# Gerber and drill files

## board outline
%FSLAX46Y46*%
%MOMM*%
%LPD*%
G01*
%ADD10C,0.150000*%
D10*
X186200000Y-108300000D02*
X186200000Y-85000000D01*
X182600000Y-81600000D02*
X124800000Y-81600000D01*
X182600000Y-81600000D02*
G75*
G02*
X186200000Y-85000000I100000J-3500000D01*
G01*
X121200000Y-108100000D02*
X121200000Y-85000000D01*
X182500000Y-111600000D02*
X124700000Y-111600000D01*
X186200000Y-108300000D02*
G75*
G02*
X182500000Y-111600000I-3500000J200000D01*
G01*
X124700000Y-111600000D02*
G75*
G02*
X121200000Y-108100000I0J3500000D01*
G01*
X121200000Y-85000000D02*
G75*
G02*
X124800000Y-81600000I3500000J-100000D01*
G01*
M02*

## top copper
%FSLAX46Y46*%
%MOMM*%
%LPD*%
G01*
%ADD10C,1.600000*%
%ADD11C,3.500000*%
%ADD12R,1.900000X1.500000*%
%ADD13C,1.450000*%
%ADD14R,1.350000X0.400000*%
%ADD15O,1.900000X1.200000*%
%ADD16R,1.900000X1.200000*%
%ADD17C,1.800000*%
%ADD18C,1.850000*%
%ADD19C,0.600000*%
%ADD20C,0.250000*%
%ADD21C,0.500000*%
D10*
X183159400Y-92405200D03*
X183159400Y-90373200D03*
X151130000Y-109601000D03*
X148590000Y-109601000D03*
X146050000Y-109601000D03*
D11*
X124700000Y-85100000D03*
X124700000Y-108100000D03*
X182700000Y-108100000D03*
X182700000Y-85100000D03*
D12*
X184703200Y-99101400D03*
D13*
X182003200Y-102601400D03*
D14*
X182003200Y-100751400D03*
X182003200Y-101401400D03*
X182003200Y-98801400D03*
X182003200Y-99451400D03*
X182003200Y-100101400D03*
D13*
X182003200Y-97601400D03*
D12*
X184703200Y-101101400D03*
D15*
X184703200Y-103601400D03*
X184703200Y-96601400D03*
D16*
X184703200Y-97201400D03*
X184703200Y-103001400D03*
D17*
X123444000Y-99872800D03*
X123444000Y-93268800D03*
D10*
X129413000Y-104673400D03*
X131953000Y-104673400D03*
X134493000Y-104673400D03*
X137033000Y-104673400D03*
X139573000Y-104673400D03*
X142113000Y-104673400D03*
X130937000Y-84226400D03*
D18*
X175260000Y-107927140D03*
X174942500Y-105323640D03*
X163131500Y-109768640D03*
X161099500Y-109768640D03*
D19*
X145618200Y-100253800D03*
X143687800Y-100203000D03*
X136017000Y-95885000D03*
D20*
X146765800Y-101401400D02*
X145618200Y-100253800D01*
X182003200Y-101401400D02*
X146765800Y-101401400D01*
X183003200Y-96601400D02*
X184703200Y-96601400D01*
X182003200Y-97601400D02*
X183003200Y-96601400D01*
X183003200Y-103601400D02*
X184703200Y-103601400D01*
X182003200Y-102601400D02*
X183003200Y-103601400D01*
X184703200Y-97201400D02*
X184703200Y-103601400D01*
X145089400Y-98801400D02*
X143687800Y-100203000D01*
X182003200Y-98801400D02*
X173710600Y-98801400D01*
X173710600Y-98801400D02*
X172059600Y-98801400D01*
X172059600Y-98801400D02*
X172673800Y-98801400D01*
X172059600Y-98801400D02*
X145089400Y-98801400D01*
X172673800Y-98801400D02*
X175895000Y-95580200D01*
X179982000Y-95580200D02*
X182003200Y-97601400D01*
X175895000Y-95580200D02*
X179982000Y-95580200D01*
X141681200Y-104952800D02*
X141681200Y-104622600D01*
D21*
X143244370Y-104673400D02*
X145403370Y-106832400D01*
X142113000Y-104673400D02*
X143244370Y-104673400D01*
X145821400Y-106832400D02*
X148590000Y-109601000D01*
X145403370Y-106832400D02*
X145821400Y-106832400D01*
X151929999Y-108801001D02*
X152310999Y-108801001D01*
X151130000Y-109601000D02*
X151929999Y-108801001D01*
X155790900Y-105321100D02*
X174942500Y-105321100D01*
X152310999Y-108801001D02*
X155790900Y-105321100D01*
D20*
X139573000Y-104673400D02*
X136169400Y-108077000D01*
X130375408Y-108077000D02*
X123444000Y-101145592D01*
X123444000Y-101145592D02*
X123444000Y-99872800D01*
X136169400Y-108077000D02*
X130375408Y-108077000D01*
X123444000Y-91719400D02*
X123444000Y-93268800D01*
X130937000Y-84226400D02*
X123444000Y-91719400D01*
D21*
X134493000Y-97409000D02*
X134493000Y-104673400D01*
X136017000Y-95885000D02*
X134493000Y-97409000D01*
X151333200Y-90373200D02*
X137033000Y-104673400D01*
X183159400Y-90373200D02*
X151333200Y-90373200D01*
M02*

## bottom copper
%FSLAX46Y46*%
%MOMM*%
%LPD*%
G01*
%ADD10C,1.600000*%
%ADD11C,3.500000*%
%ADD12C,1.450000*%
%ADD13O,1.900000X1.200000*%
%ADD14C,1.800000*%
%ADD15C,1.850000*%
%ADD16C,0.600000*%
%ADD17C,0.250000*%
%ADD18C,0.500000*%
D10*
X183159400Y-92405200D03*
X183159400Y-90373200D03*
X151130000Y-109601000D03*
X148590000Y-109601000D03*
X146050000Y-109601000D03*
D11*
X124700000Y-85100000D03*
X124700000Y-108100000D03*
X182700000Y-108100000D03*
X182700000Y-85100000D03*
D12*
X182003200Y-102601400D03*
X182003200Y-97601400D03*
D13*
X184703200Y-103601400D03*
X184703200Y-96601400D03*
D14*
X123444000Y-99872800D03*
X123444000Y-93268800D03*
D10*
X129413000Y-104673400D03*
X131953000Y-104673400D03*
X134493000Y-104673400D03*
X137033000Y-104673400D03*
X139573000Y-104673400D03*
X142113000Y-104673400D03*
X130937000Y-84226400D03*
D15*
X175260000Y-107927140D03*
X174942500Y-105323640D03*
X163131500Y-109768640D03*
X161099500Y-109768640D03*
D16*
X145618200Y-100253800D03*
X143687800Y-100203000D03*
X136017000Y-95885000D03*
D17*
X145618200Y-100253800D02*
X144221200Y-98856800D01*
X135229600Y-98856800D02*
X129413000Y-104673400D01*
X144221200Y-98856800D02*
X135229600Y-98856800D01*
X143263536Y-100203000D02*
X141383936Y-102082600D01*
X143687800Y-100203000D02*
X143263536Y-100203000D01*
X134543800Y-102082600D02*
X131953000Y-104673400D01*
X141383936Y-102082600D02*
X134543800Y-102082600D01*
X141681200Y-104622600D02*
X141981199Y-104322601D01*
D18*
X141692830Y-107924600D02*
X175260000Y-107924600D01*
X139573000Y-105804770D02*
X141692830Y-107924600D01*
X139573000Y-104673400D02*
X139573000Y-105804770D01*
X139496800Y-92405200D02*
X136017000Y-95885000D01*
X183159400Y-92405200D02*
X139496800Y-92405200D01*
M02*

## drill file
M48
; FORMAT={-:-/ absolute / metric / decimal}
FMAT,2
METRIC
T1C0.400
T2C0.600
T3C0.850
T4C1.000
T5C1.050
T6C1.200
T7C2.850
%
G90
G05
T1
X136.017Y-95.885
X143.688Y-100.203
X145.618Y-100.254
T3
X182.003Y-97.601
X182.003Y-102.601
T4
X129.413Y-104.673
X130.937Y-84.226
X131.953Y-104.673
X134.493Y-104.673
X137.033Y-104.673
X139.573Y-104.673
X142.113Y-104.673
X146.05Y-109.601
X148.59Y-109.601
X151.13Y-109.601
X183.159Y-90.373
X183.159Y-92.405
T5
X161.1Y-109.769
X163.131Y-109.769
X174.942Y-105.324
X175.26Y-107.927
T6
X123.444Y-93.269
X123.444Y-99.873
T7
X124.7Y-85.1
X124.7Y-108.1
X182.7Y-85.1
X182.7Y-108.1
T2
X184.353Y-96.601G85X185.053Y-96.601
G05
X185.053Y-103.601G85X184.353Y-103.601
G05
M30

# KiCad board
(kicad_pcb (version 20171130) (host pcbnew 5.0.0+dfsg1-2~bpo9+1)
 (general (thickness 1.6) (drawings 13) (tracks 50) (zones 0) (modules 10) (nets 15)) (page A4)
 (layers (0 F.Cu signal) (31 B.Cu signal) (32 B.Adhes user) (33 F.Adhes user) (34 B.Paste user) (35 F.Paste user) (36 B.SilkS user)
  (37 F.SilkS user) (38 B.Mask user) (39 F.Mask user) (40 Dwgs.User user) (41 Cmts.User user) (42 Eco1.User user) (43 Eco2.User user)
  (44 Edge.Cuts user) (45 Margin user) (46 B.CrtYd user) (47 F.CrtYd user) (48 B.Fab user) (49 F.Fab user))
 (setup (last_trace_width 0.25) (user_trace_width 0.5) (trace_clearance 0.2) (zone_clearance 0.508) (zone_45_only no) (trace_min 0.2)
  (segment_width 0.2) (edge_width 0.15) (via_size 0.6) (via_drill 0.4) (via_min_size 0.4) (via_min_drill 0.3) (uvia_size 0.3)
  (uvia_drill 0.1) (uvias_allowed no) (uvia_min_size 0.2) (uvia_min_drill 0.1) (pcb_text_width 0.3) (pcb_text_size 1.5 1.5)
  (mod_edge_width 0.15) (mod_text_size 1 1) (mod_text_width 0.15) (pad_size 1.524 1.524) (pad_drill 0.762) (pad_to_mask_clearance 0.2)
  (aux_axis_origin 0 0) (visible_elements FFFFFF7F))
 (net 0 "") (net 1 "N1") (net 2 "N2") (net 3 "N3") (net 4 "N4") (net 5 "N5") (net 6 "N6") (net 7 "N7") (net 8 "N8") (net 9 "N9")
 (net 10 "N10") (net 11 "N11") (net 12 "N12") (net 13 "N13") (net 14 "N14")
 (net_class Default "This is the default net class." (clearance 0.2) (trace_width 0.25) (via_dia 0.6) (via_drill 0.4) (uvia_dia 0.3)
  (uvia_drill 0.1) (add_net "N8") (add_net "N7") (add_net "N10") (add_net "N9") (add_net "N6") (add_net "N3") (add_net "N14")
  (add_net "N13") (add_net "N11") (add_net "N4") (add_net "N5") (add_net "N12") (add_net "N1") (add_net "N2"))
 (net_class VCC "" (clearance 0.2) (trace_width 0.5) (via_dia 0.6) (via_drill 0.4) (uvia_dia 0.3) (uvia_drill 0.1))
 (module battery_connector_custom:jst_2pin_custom (layer F.Cu) (at 183.1594 91.3892 90)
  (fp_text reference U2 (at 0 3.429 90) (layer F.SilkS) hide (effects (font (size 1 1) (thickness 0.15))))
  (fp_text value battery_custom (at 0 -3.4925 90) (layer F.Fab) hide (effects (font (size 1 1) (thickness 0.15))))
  (pad 1 thru_hole circle (at -1.016 0 90) (size 1.6 1.6) (drill 1) (layers *.Cu *.Mask) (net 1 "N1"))
  (pad 2 thru_hole circle (at 1.016 0 90) (size 1.6 1.6) (drill 1) (layers *.Cu *.Mask) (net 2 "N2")))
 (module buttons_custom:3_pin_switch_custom (layer F.Cu) (at 148.59 109.601 180)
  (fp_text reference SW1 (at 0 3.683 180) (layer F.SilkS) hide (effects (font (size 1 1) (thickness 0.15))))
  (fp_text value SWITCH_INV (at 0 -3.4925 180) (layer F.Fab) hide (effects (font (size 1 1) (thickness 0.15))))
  (pad 1 thru_hole circle (at -2.54 0 180) (size 1.6 1.6) (drill 1) (layers *.Cu *.Mask) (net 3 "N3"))
  (pad 2 thru_hole circle (at 0 0 180) (size 1.6 1.6) (drill 1) (layers *.Cu *.Mask) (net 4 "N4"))
  (pad 3 thru_hole circle (at 2.54 0 180) (size 1.6 1.6) (drill 1) (layers *.Cu *.Mask) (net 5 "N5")))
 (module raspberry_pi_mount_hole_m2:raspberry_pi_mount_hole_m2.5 (layer F.Cu) (at 124.7 85.1)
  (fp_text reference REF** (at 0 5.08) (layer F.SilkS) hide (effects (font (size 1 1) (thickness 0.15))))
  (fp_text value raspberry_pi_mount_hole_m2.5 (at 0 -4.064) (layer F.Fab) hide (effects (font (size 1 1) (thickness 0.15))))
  (pad 1 thru_hole circle (at 0 0) (size 3.5 3.5) (drill 2.85) (layers *.Cu *.Mask)))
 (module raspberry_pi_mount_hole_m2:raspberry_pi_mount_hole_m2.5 (layer F.Cu) (at 124.7 108.1)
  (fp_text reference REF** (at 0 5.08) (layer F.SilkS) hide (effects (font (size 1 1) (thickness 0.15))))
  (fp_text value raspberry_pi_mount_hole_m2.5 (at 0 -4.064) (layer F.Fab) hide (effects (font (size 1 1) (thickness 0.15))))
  (pad 1 thru_hole circle (at 0 0) (size 3.5 3.5) (drill 2.85) (layers *.Cu *.Mask)))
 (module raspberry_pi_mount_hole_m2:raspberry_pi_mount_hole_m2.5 (layer F.Cu) (at 182.7 108.1)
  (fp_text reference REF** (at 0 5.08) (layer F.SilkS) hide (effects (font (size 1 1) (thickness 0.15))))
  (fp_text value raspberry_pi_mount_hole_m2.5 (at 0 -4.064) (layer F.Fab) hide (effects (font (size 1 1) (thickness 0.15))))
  (pad 1 thru_hole circle (at 0 0) (size 3.5 3.5) (drill 2.85) (layers *.Cu *.Mask)))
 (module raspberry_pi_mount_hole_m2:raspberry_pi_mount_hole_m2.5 (layer F.Cu) (at 182.7 85.1)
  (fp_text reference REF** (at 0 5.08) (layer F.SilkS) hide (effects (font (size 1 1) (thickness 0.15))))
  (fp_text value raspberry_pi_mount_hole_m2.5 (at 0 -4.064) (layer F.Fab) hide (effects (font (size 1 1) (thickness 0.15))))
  (pad 1 thru_hole circle (at 0 0) (size 3.5 3.5) (drill 2.85) (layers *.Cu *.Mask)))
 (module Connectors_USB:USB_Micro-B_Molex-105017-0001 (layer F.Cu) (at 184.3532 100.1014 90)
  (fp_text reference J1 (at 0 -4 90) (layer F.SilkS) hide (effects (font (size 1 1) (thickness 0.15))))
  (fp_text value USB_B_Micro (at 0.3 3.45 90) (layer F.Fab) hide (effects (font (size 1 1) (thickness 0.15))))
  (pad 6 smd rect (at 1 0.35 90) (size 1.5 1.9) (layers F.Cu F.Paste F.Mask) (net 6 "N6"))
  (pad 6 thru_hole circle (at -2.5 -2.35 90) (size 1.45 1.45) (drill 0.85) (layers *.Cu *.Mask) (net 6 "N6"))
  (pad 2 smd rect (at -0.65 -2.35 90) (size 0.4 1.35) (layers F.Cu F.Paste F.Mask) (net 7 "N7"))
  (pad 1 smd rect (at -1.3 -2.35 90) (size 0.4 1.35) (layers F.Cu F.Paste F.Mask) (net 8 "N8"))
  (pad 5 smd rect (at 1.3 -2.35 90) (size 0.4 1.35) (layers F.Cu F.Paste F.Mask) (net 6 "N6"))
  (pad 4 smd rect (at 0.65 -2.35 90) (size 0.4 1.35) (layers F.Cu F.Paste F.Mask) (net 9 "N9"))
  (pad 3 smd rect (at 0 -2.35 90) (size 0.4 1.35) (layers F.Cu F.Paste F.Mask) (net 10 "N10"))
  (pad 6 thru_hole circle (at 2.5 -2.35 90) (size 1.45 1.45) (drill 0.85) (layers *.Cu *.Mask) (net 6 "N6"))
  (pad 6 smd rect (at -1 0.35 90) (size 1.5 1.9) (layers F.Cu F.Paste F.Mask) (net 6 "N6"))
  (pad 6 thru_hole oval (at -3.5 0.35 270) (size 1.2 1.9) (drill oval 0.6 1.3) (layers *.Cu *.Mask) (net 6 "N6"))
  (pad 6 thru_hole oval (at 3.5 0.35 90) (size 1.2 1.9) (drill oval 0.6 1.3) (layers *.Cu *.Mask) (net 6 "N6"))
  (pad 6 smd rect (at 2.9 0.35 90) (size 1.2 1.9) (layers F.Cu F.Mask) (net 6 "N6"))
  (pad 6 smd rect (at -2.9 0.35 90) (size 1.2 1.9) (layers F.Cu F.Mask) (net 6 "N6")))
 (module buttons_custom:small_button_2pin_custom (layer F.Cu) (at 123.444 96.5708 270)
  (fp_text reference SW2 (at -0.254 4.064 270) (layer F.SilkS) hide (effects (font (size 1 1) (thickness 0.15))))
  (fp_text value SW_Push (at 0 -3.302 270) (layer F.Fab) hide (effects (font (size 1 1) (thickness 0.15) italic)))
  (pad 1 thru_hole circle (at 3.302 0 270) (size 1.8 1.8) (drill 1.2) (layers *.Cu *.Mask) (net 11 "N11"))
  (pad 2 thru_hole circle (at -3.302 0 270) (size 1.8 1.8) (drill 1.2) (layers *.Cu *.Mask) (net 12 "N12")))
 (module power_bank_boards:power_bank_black (layer F.Cu) (at 135.763 104.6734)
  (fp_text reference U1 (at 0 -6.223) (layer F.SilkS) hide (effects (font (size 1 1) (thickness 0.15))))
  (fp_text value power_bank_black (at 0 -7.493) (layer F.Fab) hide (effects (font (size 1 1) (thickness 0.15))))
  (pad 1 thru_hole circle (at -6.35 0) (size 1.6 1.6) (drill 1) (layers *.Cu *.Mask) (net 8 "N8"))
  (pad 2 thru_hole circle (at -3.81 0) (size 1.6 1.6) (drill 1) (layers *.Cu *.Mask) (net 6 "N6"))
  (pad 3 thru_hole circle (at -1.27 0) (size 1.6 1.6) (drill 1) (layers *.Cu *.Mask) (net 1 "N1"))
  (pad 4 thru_hole circle (at 1.27 0) (size 1.6 1.6) (drill 1) (layers *.Cu *.Mask) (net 2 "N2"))
  (pad 5 thru_hole circle (at 3.81 0) (size 1.6 1.6) (drill 1) (layers *.Cu *.Mask) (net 11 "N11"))
  (pad 6 thru_hole circle (at 6.35 0) (size 1.6 1.6) (drill 1) (layers *.Cu *.Mask) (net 4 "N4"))
  (pad 7 thru_hole circle (at -4.826 -20.447) (size 1.6 1.6) (drill 1) (layers *.Cu *.Mask) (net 12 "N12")))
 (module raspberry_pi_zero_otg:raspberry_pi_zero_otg (layer F.Cu) (at 175.26 107.92714)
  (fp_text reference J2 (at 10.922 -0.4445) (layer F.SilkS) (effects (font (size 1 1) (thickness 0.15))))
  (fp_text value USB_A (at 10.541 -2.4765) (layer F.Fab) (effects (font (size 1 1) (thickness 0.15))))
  (pad 4 thru_hole circle (at 0 0) (size 1.85 1.85) (drill 1.05) (layers *.Cu *.Mask) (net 11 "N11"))
  (pad 1 thru_hole circle (at -0.3175 -2.6035) (size 1.85 1.85) (drill 1.05) (layers *.Cu *.Mask) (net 3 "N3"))
  (pad 3 thru_hole circle (at -12.1285 1.8415) (size 1.85 1.85) (drill 1.05) (layers *.Cu *.Mask) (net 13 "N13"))
  (pad 2 thru_hole circle (at -14.1605 1.8415) (size 1.85 1.85) (drill 1.05) (layers *.Cu *.Mask) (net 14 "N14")))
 (gr_line (start 186.2 108.3) (end 186.2 85) (angle 90) (layer Edge.Cuts) (width 0.15))
 (gr_line (start 182.6 81.6) (end 124.8 81.6) (angle 90) (layer Edge.Cuts) (width 0.15))
 (gr_arc (start 182.7 85.1) (end 182.6 81.6) (angle 90) (layer Edge.Cuts) (width 0.15))
 (gr_line (start 121.2 108.1) (end 121.2 85) (angle 90) (layer Edge.Cuts) (width 0.15))
 (gr_line (start 182.5 111.6) (end 124.7 111.6) (angle 90) (layer Edge.Cuts) (width 0.15))
 (gr_arc (start 182.7 108.1) (end 186.2 108.3) (angle 90) (layer Edge.Cuts) (width 0.15))
 (gr_arc (start 124.7 108.1) (end 124.7 111.6) (angle 90) (layer Edge.Cuts) (width 0.15))
 (gr_arc (start 124.7 85.1) (end 121.2 85) (angle 90) (layer Edge.Cuts) (width 0.15))
 (via (at 145.6182 100.2538) (size 0.6) (drill 0.4) (layers F.Cu B.Cu) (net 8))
 (segment (start 146.7658 101.4014) (end 145.6182 100.2538) (width 0.25) (layer F.Cu) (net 8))
 (segment (start 182.0032 101.4014) (end 146.7658 101.4014) (width 0.25) (layer F.Cu) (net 8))
 (segment (start 145.6182 100.2538) (end 144.2212 98.8568) (width 0.25) (layer B.Cu) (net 8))
 (segment (start 135.2296 98.8568) (end 129.413 104.6734) (width 0.25) (layer B.Cu) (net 8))
 (segment (start 144.2212 98.8568) (end 135.2296 98.8568) (width 0.25) (layer B.Cu) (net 8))
 (segment (start 183.0032 96.6014) (end 184.7032 96.6014) (width 0.25) (layer F.Cu) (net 6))
 (segment (start 182.0032 97.6014) (end 183.0032 96.6014) (width 0.25) (layer F.Cu) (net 6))
 (segment (start 183.0032 103.6014) (end 184.7032 103.6014) (width 0.25) (layer F.Cu) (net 6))
 (segment (start 182.0032 102.6014) (end 183.0032 103.6014) (width 0.25) (layer F.Cu) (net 6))
 (segment (start 184.7032 97.2014) (end 184.7032 103.6014) (width 0.25) (layer F.Cu) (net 6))
 (via (at 143.6878 100.203) (size 0.6) (drill 0.4) (layers F.Cu B.Cu) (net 6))
 (segment (start 145.0894 98.8014) (end 143.6878 100.203) (width 0.25) (layer F.Cu) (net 6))
 (segment (start 143.263536 100.203) (end 141.383936 102.0826) (width 0.25) (layer B.Cu) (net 6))
 (segment (start 143.6878 100.203) (end 143.263536 100.203) (width 0.25) (layer B.Cu) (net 6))
 (segment (start 134.5438 102.0826) (end 131.953 104.6734) (width 0.25) (layer B.Cu) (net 6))
 (segment (start 141.383936 102.0826) (end 134.5438 102.0826) (width 0.25) (layer B.Cu) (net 6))
 (segment (start 182.0032 98.8014) (end 173.7106 98.8014) (width 0.25) (layer F.Cu) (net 6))
 (segment (start 173.7106 98.8014) (end 172.0596 98.8014) (width 0.25) (layer F.Cu) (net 6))
 (segment (start 172.0596 98.8014) (end 172.6738 98.8014) (width 0.25) (layer F.Cu) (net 6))
 (segment (start 172.0596 98.8014) (end 145.0894 98.8014) (width 0.25) (layer F.Cu) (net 6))
 (segment (start 172.6738 98.8014) (end 175.895 95.5802) (width 0.25) (layer F.Cu) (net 6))
 (segment (start 179.982 95.5802) (end 182.0032 97.6014) (width 0.25) (layer F.Cu) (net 6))
 (segment (start 175.895 95.5802) (end 179.982 95.5802) (width 0.25) (layer F.Cu) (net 6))
 (segment (start 141.6812 104.9528) (end 141.6812 104.6226) (width 0.25) (layer F.Cu) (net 4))
 (segment (start 141.6812 104.6226) (end 141.981199 104.322601) (width 0.25) (layer B.Cu) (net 4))
 (segment (start 143.24437 104.6734) (end 145.40337 106.8324) (width 0.5) (layer F.Cu) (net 4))
 (segment (start 142.113 104.6734) (end 143.24437 104.6734) (width 0.5) (layer F.Cu) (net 4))
 (segment (start 145.8214 106.8324) (end 148.59 109.601) (width 0.5) (layer F.Cu) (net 4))
 (segment (start 145.40337 106.8324) (end 145.8214 106.8324) (width 0.5) (layer F.Cu) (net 4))
 (segment (start 151.929999 108.801001) (end 152.310999 108.801001) (width 0.5) (layer F.Cu) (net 3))
 (segment (start 151.13 109.601) (end 151.929999 108.801001) (width 0.5) (layer F.Cu) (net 3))
 (segment (start 155.7909 105.3211) (end 174.9425 105.3211) (width 0.5) (layer F.Cu) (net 3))
 (segment (start 152.310999 108.801001) (end 155.7909 105.3211) (width 0.5) (layer F.Cu) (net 3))
 (segment (start 139.573 104.6734) (end 136.1694 108.077) (width 0.25) (layer F.Cu) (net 11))
 (segment (start 130.375408 108.077) (end 123.444 101.145592) (width 0.25) (layer F.Cu) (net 11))
 (segment (start 123.444 101.145592) (end 123.444 99.8728) (width 0.25) (layer F.Cu) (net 11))
 (segment (start 136.1694 108.077) (end 130.375408 108.077) (width 0.25) (layer F.Cu) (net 11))
 (segment (start 141.69283 107.9246) (end 175.26 107.9246) (width 0.5) (layer B.Cu) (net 11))
 (segment (start 139.573 105.80477) (end 141.69283 107.9246) (width 0.5) (layer B.Cu) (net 11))
 (segment (start 139.573 104.6734) (end 139.573 105.80477) (width 0.5) (layer B.Cu) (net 11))
 (segment (start 123.444 91.7194) (end 123.444 93.2688) (width 0.25) (layer F.Cu) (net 12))
 (segment (start 130.937 84.2264) (end 123.444 91.7194) (width 0.25) (layer F.Cu) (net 12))
 (via (at 136.017 95.885) (size 0.6) (drill 0.4) (layers F.Cu B.Cu) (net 1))
 (segment (start 139.4968 92.4052) (end 136.017 95.885) (width 0.5) (layer B.Cu) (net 1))
 (segment (start 183.1594 92.4052) (end 139.4968 92.4052) (width 0.5) (layer B.Cu) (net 1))
 (segment (start 134.493 97.409) (end 134.493 104.6734) (width 0.5) (layer F.Cu) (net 1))
 (segment (start 136.017 95.885) (end 134.493 97.409) (width 0.5) (layer F.Cu) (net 1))
 (segment (start 151.3332 90.3732) (end 137.033 104.6734) (width 0.5) (layer F.Cu) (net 2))
 (segment (start 183.1594 90.3732) (end 151.3332 90.3732) (width 0.5) (layer F.Cu) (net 2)))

